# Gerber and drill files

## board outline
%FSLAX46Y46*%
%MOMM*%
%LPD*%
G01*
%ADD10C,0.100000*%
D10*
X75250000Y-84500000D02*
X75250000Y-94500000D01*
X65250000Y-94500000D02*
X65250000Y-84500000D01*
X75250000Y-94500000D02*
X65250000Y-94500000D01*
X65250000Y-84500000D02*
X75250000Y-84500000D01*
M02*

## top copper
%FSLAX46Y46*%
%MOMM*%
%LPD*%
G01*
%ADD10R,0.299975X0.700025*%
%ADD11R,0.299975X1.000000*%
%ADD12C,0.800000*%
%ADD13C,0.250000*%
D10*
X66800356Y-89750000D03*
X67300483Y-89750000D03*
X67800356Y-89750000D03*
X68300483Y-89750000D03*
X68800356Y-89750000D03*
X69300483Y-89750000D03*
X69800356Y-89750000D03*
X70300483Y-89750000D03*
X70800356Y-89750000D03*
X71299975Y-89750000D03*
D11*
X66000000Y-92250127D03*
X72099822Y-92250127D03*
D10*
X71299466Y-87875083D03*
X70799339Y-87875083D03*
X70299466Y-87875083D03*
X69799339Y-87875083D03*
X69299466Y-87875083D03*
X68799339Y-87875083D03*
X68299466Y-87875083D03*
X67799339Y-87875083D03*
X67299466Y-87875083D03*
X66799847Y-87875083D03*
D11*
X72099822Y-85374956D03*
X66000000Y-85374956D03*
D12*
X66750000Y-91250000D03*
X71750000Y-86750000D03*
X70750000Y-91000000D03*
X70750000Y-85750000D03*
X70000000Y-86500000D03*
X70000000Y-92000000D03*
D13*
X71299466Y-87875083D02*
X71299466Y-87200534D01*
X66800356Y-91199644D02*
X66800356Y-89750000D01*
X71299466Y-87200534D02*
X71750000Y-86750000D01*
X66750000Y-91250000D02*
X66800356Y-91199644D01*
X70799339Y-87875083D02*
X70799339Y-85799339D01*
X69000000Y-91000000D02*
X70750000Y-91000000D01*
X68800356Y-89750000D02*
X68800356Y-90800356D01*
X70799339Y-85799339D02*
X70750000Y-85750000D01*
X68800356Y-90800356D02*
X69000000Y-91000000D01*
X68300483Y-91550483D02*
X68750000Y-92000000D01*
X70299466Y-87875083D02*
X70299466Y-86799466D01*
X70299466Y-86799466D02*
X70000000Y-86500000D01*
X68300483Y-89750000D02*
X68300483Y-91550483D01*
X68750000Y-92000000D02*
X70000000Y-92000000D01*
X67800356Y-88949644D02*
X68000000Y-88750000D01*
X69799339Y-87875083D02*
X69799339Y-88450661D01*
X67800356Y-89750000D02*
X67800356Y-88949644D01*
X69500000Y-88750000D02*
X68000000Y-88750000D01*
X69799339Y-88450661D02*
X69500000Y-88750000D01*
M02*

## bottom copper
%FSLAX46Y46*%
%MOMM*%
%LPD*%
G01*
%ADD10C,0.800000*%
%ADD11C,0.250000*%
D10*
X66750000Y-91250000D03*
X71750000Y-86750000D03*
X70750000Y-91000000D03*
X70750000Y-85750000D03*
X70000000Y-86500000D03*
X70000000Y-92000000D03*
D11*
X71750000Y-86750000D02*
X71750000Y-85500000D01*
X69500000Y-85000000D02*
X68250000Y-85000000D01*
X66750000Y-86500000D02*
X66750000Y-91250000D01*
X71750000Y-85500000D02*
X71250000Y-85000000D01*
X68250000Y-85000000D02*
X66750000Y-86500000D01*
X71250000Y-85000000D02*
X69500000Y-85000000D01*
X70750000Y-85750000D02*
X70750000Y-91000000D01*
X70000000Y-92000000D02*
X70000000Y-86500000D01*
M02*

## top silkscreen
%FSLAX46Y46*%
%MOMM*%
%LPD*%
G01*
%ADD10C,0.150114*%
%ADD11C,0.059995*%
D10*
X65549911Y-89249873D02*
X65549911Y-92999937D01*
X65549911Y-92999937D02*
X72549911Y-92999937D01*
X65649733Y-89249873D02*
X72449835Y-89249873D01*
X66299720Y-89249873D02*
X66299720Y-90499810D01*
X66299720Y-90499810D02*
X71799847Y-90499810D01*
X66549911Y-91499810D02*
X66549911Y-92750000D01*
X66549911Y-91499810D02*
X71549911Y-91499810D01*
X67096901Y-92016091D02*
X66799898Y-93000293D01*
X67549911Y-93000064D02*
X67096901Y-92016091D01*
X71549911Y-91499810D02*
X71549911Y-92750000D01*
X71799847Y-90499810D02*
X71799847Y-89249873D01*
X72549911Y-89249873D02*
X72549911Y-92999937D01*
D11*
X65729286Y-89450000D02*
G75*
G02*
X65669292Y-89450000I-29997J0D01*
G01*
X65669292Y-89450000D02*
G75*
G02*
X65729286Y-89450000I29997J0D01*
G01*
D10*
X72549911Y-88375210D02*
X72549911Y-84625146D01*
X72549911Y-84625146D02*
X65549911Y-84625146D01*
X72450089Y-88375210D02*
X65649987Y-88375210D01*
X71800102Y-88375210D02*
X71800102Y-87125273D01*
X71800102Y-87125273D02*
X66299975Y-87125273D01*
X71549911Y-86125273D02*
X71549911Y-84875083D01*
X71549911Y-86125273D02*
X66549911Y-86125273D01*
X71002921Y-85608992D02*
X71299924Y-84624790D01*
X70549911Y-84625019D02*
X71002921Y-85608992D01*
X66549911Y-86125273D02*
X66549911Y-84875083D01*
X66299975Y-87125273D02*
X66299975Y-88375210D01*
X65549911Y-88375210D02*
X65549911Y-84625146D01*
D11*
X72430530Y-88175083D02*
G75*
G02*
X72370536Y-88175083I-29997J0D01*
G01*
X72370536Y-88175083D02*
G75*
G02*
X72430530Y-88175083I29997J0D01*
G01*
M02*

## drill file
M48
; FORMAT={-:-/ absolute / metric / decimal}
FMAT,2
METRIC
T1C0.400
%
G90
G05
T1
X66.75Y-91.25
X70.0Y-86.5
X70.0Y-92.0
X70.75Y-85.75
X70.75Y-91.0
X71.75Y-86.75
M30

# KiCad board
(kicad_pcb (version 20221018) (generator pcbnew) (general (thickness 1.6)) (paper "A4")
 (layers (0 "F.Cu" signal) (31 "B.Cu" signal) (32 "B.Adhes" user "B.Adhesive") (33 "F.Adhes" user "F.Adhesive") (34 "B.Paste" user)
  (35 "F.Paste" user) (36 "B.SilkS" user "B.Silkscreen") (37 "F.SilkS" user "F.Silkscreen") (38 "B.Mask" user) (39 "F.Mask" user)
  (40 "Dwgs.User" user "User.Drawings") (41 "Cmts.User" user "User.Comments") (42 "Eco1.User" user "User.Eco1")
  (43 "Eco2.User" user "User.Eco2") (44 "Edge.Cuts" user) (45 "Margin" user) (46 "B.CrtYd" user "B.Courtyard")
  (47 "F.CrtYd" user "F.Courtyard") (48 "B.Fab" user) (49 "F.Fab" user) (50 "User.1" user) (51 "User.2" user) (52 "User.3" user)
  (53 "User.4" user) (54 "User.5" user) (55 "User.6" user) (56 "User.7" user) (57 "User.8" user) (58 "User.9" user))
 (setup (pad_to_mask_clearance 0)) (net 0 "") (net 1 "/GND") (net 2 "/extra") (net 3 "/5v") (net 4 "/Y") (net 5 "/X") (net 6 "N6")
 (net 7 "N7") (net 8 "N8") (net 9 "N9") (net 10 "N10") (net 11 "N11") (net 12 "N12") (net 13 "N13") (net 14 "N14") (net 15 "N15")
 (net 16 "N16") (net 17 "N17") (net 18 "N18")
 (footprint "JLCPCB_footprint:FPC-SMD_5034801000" (layer "F.Cu") (at 69.049911 91.125083)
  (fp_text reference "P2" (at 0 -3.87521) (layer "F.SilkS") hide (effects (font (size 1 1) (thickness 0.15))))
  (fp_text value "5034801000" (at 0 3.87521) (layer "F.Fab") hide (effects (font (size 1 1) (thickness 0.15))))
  (fp_line (start -3.5 -1.87521) (end -3.5 1.874854) (stroke (width 0.150114) (type solid)) (layer "F.SilkS"))
  (fp_line (start -3.5 1.874854) (end 3.5 1.874854) (stroke (width 0.150114) (type solid)) (layer "F.SilkS"))
  (fp_line (start -3.400178 -1.87521) (end 3.399924 -1.87521) (stroke (width 0.150114) (type solid)) (layer "F.SilkS"))
  (fp_line (start -2.750191 -1.87521) (end -2.750191 -0.625273) (stroke (width 0.150114) (type solid)) (layer "F.SilkS"))
  (fp_line (start -2.750191 -0.625273) (end 2.749936 -0.625273) (stroke (width 0.150114) (type solid)) (layer "F.SilkS"))
  (fp_line (start -2.5 0.374727) (end -2.5 1.624917) (stroke (width 0.150114) (type solid)) (layer "F.SilkS"))
  (fp_line (start -2.5 0.374727) (end 2.5 0.374727) (stroke (width 0.150114) (type solid)) (layer "F.SilkS"))
  (fp_line (start -1.95301 0.891008) (end -2.250013 1.87521) (stroke (width 0.150114) (type solid)) (layer "F.SilkS"))
  (fp_line (start -1.5 1.874981) (end -1.95301 0.891008) (stroke (width 0.150114) (type solid)) (layer "F.SilkS"))
  (fp_line (start 2.5 0.374727) (end 2.5 1.624917) (stroke (width 0.150114) (type solid)) (layer "F.SilkS"))
  (fp_line (start 2.749936 -0.625273) (end 2.749936 -1.87521) (stroke (width 0.150114) (type solid)) (layer "F.SilkS"))
  (fp_line (start 3.5 -1.87521) (end 3.5 1.874854) (stroke (width 0.150114) (type solid)) (layer "F.SilkS"))
  (fp_circle (center -3.350622 -1.675083) (end -3.320625 -1.675083) (stroke (width 0.059995) (type solid)) (fill none) (layer "F.SilkS"))
  (pad "1" smd rect (at -2.249555 -1.375083 180) (size 0.299975 0.700025) (layers "F.Cu" "F.Paste" "F.Mask") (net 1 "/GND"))
  (pad "2" smd rect (at -1.749428 -1.375083 180) (size 0.299975 0.700025) (layers "F.Cu" "F.Paste" "F.Mask") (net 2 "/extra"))
  (pad "3" smd rect (at -1.249555 -1.375083 180) (size 0.299975 0.700025) (layers "F.Cu" "F.Paste" "F.Mask") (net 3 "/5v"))
  (pad "4" smd rect (at -0.749428 -1.375083 180) (size 0.299975 0.700025) (layers "F.Cu" "F.Paste" "F.Mask") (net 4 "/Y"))
  (pad "5" smd rect (at -0.249555 -1.375083 180) (size 0.299975 0.700025) (layers "F.Cu" "F.Paste" "F.Mask") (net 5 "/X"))
  (pad "6" smd rect (at 0.250572 -1.375083 180) (size 0.299975 0.700025) (layers "F.Cu" "F.Paste" "F.Mask") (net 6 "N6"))
  (pad "7" smd rect (at 0.750445 -1.375083 180) (size 0.299975 0.700025) (layers "F.Cu" "F.Paste" "F.Mask") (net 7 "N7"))
  (pad "8" smd rect (at 1.250572 -1.375083 180) (size 0.299975 0.700025) (layers "F.Cu" "F.Paste" "F.Mask") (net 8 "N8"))
  (pad "9" smd rect (at 1.750445 -1.375083 180) (size 0.299975 0.700025) (layers "F.Cu" "F.Paste" "F.Mask") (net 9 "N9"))
  (pad "10" smd rect (at 2.250064 -1.375083 180) (size 0.299975 0.700025) (layers "F.Cu" "F.Paste" "F.Mask") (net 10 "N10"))
  (pad "11" smd rect (at -3.049911 1.125044) (size 0.299975 1) (layers "F.Cu" "F.Paste" "F.Mask") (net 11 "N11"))
  (pad "12" smd rect (at 3.049911 1.125044 180) (size 0.299975 1) (layers "F.Cu" "F.Paste" "F.Mask") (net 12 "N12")))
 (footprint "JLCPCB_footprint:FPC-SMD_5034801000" (layer "F.Cu") (at 69.049911 86.5 180)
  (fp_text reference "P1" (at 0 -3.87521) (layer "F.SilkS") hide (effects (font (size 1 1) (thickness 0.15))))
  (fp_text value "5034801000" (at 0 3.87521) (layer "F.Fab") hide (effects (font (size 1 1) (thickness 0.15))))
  (fp_line (start -3.5 -1.87521) (end -3.5 1.874854) (stroke (width 0.150114) (type solid)) (layer "F.SilkS"))
  (fp_line (start -3.5 1.874854) (end 3.5 1.874854) (stroke (width 0.150114) (type solid)) (layer "F.SilkS"))
  (fp_line (start -3.400178 -1.87521) (end 3.399924 -1.87521) (stroke (width 0.150114) (type solid)) (layer "F.SilkS"))
  (fp_line (start -2.750191 -1.87521) (end -2.750191 -0.625273) (stroke (width 0.150114) (type solid)) (layer "F.SilkS"))
  (fp_line (start -2.750191 -0.625273) (end 2.749936 -0.625273) (stroke (width 0.150114) (type solid)) (layer "F.SilkS"))
  (fp_line (start -2.5 0.374727) (end -2.5 1.624917) (stroke (width 0.150114) (type solid)) (layer "F.SilkS"))
  (fp_line (start -2.5 0.374727) (end 2.5 0.374727) (stroke (width 0.150114) (type solid)) (layer "F.SilkS"))
  (fp_line (start -1.95301 0.891008) (end -2.250013 1.87521) (stroke (width 0.150114) (type solid)) (layer "F.SilkS"))
  (fp_line (start -1.5 1.874981) (end -1.95301 0.891008) (stroke (width 0.150114) (type solid)) (layer "F.SilkS"))
  (fp_line (start 2.5 0.374727) (end 2.5 1.624917) (stroke (width 0.150114) (type solid)) (layer "F.SilkS"))
  (fp_line (start 2.749936 -0.625273) (end 2.749936 -1.87521) (stroke (width 0.150114) (type solid)) (layer "F.SilkS"))
  (fp_line (start 3.5 -1.87521) (end 3.5 1.874854) (stroke (width 0.150114) (type solid)) (layer "F.SilkS"))
  (fp_circle (center -3.350622 -1.675083) (end -3.320625 -1.675083) (stroke (width 0.059995) (type solid)) (fill none) (layer "F.SilkS"))
  (pad "1" smd rect (at -2.249555 -1.375083) (size 0.299975 0.700025) (layers "F.Cu" "F.Paste" "F.Mask") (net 1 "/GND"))
  (pad "2" smd rect (at -1.749428 -1.375083) (size 0.299975 0.700025) (layers "F.Cu" "F.Paste" "F.Mask") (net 5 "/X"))
  (pad "3" smd rect (at -1.249555 -1.375083) (size 0.299975 0.700025) (layers "F.Cu" "F.Paste" "F.Mask") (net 4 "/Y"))
  (pad "4" smd rect (at -0.749428 -1.375083) (size 0.299975 0.700025) (layers "F.Cu" "F.Paste" "F.Mask") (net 3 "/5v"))
  (pad "5" smd rect (at -0.249555 -1.375083) (size 0.299975 0.700025) (layers "F.Cu" "F.Paste" "F.Mask") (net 3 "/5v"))
  (pad "6" smd rect (at 0.250572 -1.375083) (size 0.299975 0.700025) (layers "F.Cu" "F.Paste" "F.Mask") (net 3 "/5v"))
  (pad "7" smd rect (at 0.750445 -1.375083) (size 0.299975 0.700025) (layers "F.Cu" "F.Paste" "F.Mask") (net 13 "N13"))
  (pad "8" smd rect (at 1.250572 -1.375083) (size 0.299975 0.700025) (layers "F.Cu" "F.Paste" "F.Mask") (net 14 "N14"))
  (pad "9" smd rect (at 1.750445 -1.375083) (size 0.299975 0.700025) (layers "F.Cu" "F.Paste" "F.Mask") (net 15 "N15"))
  (pad "10" smd rect (at 2.250064 -1.375083) (size 0.299975 0.700025) (layers "F.Cu" "F.Paste" "F.Mask") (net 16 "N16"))
  (pad "11" smd rect (at -3.049911 1.125044 180) (size 0.299975 1) (layers "F.Cu" "F.Paste" "F.Mask") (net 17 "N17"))
  (pad "12" smd rect (at 3.049911 1.125044) (size 0.299975 1) (layers "F.Cu" "F.Paste" "F.Mask") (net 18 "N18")))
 (gr_line (start 75.25 84.5) (end 75.25 94.5) (stroke (width 0.1) (type default)) (layer "Edge.Cuts"))
 (gr_line (start 65.25 94.5) (end 65.25 84.5) (stroke (width 0.1) (type default)) (layer "Edge.Cuts"))
 (gr_line (start 75.25 94.5) (end 65.25 94.5) (stroke (width 0.1) (type default)) (layer "Edge.Cuts"))
 (gr_line (start 65.25 84.5) (end 75.25 84.5) (stroke (width 0.1) (type default)) (layer "Edge.Cuts"))
 (segment (start 71.299466 87.875083) (end 71.299466 87.200534) (width 0.25) (layer "F.Cu") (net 1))
 (segment (start 66.800356 91.199644) (end 66.800356 89.75) (width 0.25) (layer "F.Cu") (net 1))
 (segment (start 71.299466 87.200534) (end 71.75 86.75) (width 0.25) (layer "F.Cu") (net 1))
 (segment (start 66.75 91.25) (end 66.800356 91.199644) (width 0.25) (layer "F.Cu") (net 1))
 (via (at 66.75 91.25) (size 0.8) (drill 0.4) (layers "F.Cu" "B.Cu") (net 1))
 (via (at 71.75 86.75) (size 0.8) (drill 0.4) (layers "F.Cu" "B.Cu") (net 1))
 (segment (start 71.75 86.75) (end 71.75 85.5) (width 0.25) (layer "B.Cu") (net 1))
 (segment (start 69.5 85) (end 68.25 85) (width 0.25) (layer "B.Cu") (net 1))
 (segment (start 66.75 86.5) (end 66.75 91.25) (width 0.25) (layer "B.Cu") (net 1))
 (segment (start 71.75 85.5) (end 71.25 85) (width 0.25) (layer "B.Cu") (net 1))
 (segment (start 68.25 85) (end 66.75 86.5) (width 0.25) (layer "B.Cu") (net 1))
 (segment (start 71.25 85) (end 69.5 85) (width 0.25) (layer "B.Cu") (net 1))
 (segment (start 70.799339 87.875083) (end 70.799339 85.799339) (width 0.25) (layer "F.Cu") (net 5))
 (segment (start 69 91) (end 70.75 91) (width 0.25) (layer "F.Cu") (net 5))
 (segment (start 68.800356 89.75) (end 68.800356 90.800356) (width 0.25) (layer "F.Cu") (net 5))
 (segment (start 70.799339 85.799339) (end 70.75 85.75) (width 0.25) (layer "F.Cu") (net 5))
 (segment (start 68.800356 90.800356) (end 69 91) (width 0.25) (layer "F.Cu") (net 5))
 (via (at 70.75 91) (size 0.8) (drill 0.4) (layers "F.Cu" "B.Cu") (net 5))
 (via (at 70.75 85.75) (size 0.8) (drill 0.4) (layers "F.Cu" "B.Cu") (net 5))
 (segment (start 70.75 85.75) (end 70.75 91) (width 0.25) (layer "B.Cu") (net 5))
 (segment (start 68.300483 91.550483) (end 68.75 92) (width 0.25) (layer "F.Cu") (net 4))
 (segment (start 70.299466 87.875083) (end 70.299466 86.799466) (width 0.25) (layer "F.Cu") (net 4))
 (segment (start 70.299466 86.799466) (end 70 86.5) (width 0.25) (layer "F.Cu") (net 4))
 (segment (start 68.300483 89.75) (end 68.300483 91.550483) (width 0.25) (layer "F.Cu") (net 4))
 (segment (start 68.75 92) (end 70 92) (width 0.25) (layer "F.Cu") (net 4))
 (via (at 70 86.5) (size 0.8) (drill 0.4) (layers "F.Cu" "B.Cu") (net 4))
 (via (at 70 92) (size 0.8) (drill 0.4) (layers "F.Cu" "B.Cu") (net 4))
 (segment (start 70 92) (end 70 86.5) (width 0.25) (layer "B.Cu") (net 4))
 (segment (start 67.800356 88.949644) (end 68 88.75) (width 0.25) (layer "F.Cu") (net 3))
 (segment (start 69.799339 87.875083) (end 69.799339 88.450661) (width 0.25) (layer "F.Cu") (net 3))
 (segment (start 67.800356 89.75) (end 67.800356 88.949644) (width 0.25) (layer "F.Cu") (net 3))
 (segment (start 69.5 88.75) (end 68 88.75) (width 0.25) (layer "F.Cu") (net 3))
 (segment (start 69.799339 88.450661) (end 69.5 88.75) (width 0.25) (layer "F.Cu") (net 3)))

